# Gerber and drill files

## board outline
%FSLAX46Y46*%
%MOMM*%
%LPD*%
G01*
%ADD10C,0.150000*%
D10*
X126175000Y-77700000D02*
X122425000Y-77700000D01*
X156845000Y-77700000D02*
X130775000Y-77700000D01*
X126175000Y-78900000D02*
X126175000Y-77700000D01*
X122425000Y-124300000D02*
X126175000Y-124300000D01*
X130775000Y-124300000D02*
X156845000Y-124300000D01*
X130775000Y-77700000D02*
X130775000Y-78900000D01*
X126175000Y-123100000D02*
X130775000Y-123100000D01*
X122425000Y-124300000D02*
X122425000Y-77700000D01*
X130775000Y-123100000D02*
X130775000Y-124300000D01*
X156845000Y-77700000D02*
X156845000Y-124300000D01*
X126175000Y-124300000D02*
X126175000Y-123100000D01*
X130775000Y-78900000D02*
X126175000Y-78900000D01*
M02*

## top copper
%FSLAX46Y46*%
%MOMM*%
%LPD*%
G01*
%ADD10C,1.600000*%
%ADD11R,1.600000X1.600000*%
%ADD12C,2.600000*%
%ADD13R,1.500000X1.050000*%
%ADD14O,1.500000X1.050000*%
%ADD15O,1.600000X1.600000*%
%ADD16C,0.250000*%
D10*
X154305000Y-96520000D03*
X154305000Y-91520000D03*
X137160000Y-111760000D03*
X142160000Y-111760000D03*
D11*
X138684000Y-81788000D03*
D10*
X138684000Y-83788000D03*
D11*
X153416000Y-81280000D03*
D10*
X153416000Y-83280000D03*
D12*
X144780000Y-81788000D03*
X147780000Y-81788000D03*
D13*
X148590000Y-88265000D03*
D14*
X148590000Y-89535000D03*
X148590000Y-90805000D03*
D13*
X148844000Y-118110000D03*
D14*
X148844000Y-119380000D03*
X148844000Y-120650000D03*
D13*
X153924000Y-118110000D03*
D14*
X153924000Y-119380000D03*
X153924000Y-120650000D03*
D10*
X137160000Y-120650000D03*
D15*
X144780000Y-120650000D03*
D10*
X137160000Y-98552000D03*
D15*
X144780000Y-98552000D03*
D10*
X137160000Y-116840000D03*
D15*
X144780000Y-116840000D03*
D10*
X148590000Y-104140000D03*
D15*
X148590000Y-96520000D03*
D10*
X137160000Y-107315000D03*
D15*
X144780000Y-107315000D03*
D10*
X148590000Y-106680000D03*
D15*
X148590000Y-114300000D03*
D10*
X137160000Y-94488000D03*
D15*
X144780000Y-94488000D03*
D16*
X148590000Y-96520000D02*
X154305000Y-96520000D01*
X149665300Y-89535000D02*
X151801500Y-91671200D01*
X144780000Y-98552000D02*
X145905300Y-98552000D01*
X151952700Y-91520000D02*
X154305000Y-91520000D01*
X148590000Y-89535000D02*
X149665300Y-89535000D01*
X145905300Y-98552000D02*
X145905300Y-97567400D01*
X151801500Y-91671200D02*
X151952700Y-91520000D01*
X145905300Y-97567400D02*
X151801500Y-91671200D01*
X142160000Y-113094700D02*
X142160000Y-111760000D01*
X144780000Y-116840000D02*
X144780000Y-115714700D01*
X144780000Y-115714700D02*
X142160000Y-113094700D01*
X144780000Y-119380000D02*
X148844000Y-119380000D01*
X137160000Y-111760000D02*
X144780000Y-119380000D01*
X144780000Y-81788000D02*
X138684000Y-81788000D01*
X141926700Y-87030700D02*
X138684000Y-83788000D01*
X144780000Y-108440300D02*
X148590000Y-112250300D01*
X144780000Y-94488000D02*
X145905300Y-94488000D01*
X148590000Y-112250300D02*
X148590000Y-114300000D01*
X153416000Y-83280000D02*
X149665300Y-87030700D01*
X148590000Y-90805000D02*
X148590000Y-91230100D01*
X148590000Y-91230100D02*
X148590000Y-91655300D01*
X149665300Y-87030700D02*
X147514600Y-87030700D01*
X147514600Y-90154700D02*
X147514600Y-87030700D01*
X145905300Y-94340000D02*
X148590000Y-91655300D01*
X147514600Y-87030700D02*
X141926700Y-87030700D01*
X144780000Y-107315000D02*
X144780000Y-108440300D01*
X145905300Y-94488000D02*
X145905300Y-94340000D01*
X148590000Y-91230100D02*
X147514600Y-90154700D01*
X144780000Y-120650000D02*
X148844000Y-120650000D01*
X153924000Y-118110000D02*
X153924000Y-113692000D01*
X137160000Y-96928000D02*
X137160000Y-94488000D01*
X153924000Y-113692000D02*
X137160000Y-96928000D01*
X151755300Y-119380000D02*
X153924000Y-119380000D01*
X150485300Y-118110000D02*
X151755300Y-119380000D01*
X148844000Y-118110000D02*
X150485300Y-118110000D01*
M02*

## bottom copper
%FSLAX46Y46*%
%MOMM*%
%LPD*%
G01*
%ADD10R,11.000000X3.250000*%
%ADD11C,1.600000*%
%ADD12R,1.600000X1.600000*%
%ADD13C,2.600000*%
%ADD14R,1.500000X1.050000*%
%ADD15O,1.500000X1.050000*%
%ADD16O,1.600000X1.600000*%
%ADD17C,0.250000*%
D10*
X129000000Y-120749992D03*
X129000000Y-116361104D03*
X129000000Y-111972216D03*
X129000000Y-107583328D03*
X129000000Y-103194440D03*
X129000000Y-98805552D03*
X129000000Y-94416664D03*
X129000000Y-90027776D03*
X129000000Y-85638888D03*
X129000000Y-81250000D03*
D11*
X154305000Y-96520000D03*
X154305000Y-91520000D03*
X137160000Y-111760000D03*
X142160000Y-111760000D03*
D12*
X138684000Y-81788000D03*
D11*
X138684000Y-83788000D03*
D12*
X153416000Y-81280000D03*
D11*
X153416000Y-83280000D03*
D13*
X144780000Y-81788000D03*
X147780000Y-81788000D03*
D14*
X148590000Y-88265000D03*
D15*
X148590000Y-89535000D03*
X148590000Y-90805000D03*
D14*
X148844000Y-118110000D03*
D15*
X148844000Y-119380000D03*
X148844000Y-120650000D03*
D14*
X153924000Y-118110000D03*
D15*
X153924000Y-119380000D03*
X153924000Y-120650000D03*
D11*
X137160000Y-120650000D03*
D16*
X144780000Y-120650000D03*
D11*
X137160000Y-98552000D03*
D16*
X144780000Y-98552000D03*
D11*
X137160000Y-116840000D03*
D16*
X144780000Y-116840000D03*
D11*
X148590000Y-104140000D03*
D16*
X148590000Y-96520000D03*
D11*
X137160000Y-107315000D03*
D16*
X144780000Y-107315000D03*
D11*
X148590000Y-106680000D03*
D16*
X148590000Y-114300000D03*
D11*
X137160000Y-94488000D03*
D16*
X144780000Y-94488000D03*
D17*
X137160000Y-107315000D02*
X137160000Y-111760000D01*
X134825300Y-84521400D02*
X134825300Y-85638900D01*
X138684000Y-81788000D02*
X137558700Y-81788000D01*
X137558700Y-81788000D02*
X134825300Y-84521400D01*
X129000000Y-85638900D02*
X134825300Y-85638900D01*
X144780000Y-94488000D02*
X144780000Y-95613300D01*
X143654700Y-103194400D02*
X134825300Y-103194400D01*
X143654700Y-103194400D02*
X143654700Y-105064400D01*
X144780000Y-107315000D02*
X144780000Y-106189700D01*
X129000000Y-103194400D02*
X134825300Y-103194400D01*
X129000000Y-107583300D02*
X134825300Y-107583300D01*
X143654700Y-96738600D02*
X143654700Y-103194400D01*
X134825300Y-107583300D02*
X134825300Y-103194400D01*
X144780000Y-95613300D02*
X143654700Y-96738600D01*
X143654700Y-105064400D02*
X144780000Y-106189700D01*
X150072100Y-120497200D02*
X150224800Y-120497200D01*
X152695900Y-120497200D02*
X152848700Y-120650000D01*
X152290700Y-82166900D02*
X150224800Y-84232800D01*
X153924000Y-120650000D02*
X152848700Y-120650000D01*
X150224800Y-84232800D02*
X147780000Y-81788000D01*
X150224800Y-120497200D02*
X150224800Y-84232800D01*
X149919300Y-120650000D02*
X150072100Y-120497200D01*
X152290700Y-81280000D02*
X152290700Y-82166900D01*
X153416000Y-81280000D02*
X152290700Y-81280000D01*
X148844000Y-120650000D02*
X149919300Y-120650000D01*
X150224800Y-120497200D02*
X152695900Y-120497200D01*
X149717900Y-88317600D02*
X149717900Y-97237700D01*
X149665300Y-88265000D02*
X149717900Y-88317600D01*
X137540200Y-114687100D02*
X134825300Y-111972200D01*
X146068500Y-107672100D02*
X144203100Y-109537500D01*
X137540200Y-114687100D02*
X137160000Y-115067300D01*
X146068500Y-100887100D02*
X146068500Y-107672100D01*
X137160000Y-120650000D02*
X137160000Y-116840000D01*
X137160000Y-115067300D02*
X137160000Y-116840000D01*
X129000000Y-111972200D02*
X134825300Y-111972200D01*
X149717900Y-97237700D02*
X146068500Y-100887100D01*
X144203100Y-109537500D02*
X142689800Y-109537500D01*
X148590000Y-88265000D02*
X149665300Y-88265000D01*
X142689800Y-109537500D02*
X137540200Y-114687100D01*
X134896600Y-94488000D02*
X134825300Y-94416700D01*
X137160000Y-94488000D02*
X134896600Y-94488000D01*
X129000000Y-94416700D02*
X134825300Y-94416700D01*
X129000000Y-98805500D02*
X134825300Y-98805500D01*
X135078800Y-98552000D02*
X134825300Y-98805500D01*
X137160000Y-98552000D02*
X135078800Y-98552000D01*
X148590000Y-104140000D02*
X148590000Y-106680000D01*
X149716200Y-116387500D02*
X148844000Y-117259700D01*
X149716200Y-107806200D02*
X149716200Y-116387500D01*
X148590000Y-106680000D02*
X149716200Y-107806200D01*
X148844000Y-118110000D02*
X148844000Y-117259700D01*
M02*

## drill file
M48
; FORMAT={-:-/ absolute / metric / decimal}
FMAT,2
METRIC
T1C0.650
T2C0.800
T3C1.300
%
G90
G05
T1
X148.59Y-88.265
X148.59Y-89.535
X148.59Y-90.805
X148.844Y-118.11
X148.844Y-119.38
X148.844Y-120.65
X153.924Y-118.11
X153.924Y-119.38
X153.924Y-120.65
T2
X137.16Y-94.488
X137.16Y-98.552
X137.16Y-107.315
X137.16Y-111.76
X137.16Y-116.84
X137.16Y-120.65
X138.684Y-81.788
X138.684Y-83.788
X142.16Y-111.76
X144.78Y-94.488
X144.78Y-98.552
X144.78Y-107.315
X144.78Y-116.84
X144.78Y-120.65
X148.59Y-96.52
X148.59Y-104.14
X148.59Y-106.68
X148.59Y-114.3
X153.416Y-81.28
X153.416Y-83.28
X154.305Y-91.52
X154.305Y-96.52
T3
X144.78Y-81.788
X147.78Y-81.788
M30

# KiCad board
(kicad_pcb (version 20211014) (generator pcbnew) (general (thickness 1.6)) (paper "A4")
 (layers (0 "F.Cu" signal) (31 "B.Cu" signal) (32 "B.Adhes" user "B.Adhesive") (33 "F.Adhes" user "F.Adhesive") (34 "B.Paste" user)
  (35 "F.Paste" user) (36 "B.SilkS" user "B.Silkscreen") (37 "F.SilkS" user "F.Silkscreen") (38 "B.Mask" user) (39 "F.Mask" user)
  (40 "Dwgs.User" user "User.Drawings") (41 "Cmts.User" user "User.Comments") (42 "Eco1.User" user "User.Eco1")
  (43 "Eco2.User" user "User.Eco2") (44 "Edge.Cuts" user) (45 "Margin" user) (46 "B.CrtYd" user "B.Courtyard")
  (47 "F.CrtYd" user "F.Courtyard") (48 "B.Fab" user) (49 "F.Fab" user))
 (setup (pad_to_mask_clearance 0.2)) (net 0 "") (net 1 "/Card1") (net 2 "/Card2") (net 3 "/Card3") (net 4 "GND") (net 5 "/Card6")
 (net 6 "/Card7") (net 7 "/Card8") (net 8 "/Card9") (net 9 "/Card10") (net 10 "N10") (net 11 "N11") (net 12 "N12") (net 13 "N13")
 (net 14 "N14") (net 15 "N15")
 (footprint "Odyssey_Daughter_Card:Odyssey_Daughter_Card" (layer "F.Cu") (at 129 101)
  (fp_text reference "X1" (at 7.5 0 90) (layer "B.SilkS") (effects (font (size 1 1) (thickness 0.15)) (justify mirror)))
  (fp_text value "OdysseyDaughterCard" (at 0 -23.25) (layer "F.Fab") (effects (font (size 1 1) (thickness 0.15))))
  (pad "1" smd rect locked (at 0 19.749992) (size 11 3.25) (layers "B.Cu" "B.Mask") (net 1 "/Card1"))
  (pad "2" smd rect locked (at 0 15.361104) (size 11 3.25) (layers "B.Cu" "B.Mask") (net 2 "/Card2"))
  (pad "3" smd rect locked (at 0 10.972216) (size 11 3.25) (layers "B.Cu" "B.Mask") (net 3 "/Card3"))
  (pad "4" smd rect locked (at 0 6.583328) (size 11 3.25) (layers "B.Cu" "B.Mask") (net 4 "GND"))
  (pad "5" smd rect locked (at 0 2.19444) (size 11 3.25) (layers "B.Cu" "B.Mask") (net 4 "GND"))
  (pad "6" smd rect locked (at 0 -2.194448) (size 11 3.25) (layers "B.Cu" "B.Mask") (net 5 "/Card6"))
  (pad "7" smd rect locked (at 0 -6.583336) (size 11 3.25) (layers "B.Cu" "B.Mask") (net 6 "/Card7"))
  (pad "8" smd rect locked (at 0 -10.972224) (size 11 3.25) (layers "B.Cu" "B.Mask") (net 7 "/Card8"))
  (pad "9" smd rect locked (at 0 -15.361112) (size 11 3.25) (layers "B.Cu" "B.Mask") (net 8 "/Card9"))
  (pad "10" smd rect locked (at 0 -19.75) (size 11 3.25) (layers "B.Cu" "B.Mask") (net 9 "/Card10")))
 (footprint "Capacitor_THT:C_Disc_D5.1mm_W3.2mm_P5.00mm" (layer "F.Cu") (at 154.305 96.52 90)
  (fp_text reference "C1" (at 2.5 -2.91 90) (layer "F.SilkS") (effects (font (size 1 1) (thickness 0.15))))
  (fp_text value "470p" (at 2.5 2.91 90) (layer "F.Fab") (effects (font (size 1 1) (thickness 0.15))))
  (pad "1" thru_hole circle locked (at 0 0 90) (size 1.6 1.6) (drill 0.8) (layers *.Cu *.Mask) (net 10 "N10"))
  (pad "2" thru_hole circle locked (at 5 0 90) (size 1.6 1.6) (drill 0.8) (layers *.Cu *.Mask) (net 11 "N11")))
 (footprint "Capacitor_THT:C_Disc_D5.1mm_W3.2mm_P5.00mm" (layer "F.Cu") (at 137.16 111.76)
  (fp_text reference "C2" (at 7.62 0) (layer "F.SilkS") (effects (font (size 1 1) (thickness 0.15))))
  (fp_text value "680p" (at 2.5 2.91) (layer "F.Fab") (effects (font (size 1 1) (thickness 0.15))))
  (pad "1" thru_hole circle locked (at 0 0) (size 1.6 1.6) (drill 0.8) (layers *.Cu *.Mask) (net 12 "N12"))
  (pad "2" thru_hole circle locked (at 5 0) (size 1.6 1.6) (drill 0.8) (layers *.Cu *.Mask) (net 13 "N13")))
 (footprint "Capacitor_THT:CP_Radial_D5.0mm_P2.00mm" (layer "F.Cu") (at 138.684 81.788 -90)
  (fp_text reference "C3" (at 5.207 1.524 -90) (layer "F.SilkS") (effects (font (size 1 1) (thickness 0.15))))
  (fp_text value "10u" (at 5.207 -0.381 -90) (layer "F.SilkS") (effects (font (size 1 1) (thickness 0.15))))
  (pad "1" thru_hole rect locked (at 0 0 270) (size 1.6 1.6) (drill 0.8) (layers *.Cu *.Mask) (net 8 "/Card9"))
  (pad "2" thru_hole circle locked (at 2 0 270) (size 1.6 1.6) (drill 0.8) (layers *.Cu *.Mask) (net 4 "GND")))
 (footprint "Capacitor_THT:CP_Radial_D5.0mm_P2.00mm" (layer "F.Cu") (at 153.416 81.28 -90)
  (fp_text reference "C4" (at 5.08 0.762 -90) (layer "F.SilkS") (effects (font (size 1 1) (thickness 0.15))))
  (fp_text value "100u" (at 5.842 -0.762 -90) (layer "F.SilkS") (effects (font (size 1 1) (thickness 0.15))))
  (pad "1" thru_hole rect locked (at 0 0 270) (size 1.6 1.6) (drill 0.8) (layers *.Cu *.Mask) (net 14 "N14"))
  (pad "2" thru_hole circle locked (at 2 0 270) (size 1.6 1.6) (drill 0.8) (layers *.Cu *.Mask) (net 4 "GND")))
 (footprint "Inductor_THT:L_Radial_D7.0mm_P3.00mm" (layer "F.Cu") (at 144.78 81.788)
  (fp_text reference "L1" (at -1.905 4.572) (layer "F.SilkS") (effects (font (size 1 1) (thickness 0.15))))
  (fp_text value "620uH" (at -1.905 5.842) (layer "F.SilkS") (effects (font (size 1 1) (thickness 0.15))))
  (pad "1" thru_hole circle locked (at 0 0) (size 2.6 2.6) (drill 1.3) (layers *.Cu *.Mask) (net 8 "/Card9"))
  (pad "2" thru_hole circle locked (at 3 0) (size 2.6 2.6) (drill 1.3) (layers *.Cu *.Mask) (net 14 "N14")))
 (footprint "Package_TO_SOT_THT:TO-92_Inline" (layer "F.Cu") (at 148.59 88.265 -90)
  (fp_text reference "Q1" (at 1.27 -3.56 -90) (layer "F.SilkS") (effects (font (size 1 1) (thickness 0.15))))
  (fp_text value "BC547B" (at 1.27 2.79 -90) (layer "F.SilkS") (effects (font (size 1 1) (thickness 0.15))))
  (pad "1" thru_hole rect locked (at 0 0 270) (size 1.05 1.5) (drill 0.65) (layers *.Cu *.Mask) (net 3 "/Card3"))
  (pad "2" thru_hole oval locked (at 1.27 0 270) (size 1.05 1.5) (drill 0.65) (layers *.Cu *.Mask) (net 11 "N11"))
  (pad "3" thru_hole oval locked (at 2.54 0 270) (size 1.05 1.5) (drill 0.65) (layers *.Cu *.Mask) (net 4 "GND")))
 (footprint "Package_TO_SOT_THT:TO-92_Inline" (layer "F.Cu") (at 148.844 118.11 -90)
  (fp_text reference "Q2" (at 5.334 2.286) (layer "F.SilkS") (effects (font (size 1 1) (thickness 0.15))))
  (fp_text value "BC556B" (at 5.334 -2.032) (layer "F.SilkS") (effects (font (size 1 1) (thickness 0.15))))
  (pad "1" thru_hole rect locked (at 0 0 270) (size 1.05 1.5) (drill 0.65) (layers *.Cu *.Mask) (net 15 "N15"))
  (pad "2" thru_hole oval locked (at 1.27 0 270) (size 1.05 1.5) (drill 0.65) (layers *.Cu *.Mask) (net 12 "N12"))
  (pad "3" thru_hole oval locked (at 2.54 0 270) (size 1.05 1.5) (drill 0.65) (layers *.Cu *.Mask) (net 14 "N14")))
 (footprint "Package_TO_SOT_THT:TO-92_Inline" (layer "F.Cu") (at 153.924 118.11 -90)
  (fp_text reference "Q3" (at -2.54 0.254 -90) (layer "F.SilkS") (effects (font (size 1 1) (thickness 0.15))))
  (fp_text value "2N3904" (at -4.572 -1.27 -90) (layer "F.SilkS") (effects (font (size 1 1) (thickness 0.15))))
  (pad "1" thru_hole rect locked (at 0 0 270) (size 1.05 1.5) (drill 0.65) (layers *.Cu *.Mask) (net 6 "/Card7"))
  (pad "2" thru_hole oval locked (at 1.27 0 270) (size 1.05 1.5) (drill 0.65) (layers *.Cu *.Mask) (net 15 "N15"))
  (pad "3" thru_hole oval locked (at 2.54 0 270) (size 1.05 1.5) (drill 0.65) (layers *.Cu *.Mask) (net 14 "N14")))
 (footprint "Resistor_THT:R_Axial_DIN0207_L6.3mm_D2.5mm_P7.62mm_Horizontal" (layer "F.Cu") (at 137.16 120.65)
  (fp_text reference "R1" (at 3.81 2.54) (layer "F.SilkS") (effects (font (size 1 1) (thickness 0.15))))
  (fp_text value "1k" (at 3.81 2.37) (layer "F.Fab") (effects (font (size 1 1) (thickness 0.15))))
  (pad "1" thru_hole circle locked (at 0 0) (size 1.6 1.6) (drill 0.8) (layers *.Cu *.Mask) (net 3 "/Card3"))
  (pad "2" thru_hole oval locked (at 7.62 0) (size 1.6 1.6) (drill 0.8) (layers *.Cu *.Mask) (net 14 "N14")))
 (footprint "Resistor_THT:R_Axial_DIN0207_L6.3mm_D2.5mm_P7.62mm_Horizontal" (layer "F.Cu") (at 137.16 98.552)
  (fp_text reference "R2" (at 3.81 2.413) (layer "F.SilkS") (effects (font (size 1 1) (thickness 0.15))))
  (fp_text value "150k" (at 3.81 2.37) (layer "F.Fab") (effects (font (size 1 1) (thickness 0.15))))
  (pad "1" thru_hole circle locked (at 0 0) (size 1.6 1.6) (drill 0.8) (layers *.Cu *.Mask) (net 5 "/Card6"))
  (pad "2" thru_hole oval locked (at 7.62 0) (size 1.6 1.6) (drill 0.8) (layers *.Cu *.Mask) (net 11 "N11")))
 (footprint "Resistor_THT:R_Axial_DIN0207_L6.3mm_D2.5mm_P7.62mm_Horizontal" (layer "F.Cu") (at 137.16 116.84)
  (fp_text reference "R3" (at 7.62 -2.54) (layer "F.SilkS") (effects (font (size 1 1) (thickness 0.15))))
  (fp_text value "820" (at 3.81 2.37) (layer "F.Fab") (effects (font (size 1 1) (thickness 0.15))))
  (pad "1" thru_hole circle locked (at 0 0) (size 1.6 1.6) (drill 0.8) (layers *.Cu *.Mask) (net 3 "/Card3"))
  (pad "2" thru_hole oval locked (at 7.62 0) (size 1.6 1.6) (drill 0.8) (layers *.Cu *.Mask) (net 13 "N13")))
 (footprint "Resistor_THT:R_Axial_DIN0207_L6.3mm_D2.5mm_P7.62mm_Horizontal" (layer "F.Cu") (at 148.59 104.14 90)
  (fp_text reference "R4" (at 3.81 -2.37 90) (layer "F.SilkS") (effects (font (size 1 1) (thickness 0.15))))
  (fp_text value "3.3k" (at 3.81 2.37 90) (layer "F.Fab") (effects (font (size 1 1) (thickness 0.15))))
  (pad "1" thru_hole circle locked (at 0 0 90) (size 1.6 1.6) (drill 0.8) (layers *.Cu *.Mask) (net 15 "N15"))
  (pad "2" thru_hole oval locked (at 7.62 0 90) (size 1.6 1.6) (drill 0.8) (layers *.Cu *.Mask) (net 10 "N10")))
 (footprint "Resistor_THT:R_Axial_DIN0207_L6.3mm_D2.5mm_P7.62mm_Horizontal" (layer "F.Cu") (at 137.16 107.315)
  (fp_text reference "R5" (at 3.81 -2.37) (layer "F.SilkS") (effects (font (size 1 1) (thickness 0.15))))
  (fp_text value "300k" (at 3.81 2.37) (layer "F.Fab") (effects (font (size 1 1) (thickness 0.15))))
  (pad "1" thru_hole circle locked (at 0 0) (size 1.6 1.6) (drill 0.8) (layers *.Cu *.Mask) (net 12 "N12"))
  (pad "2" thru_hole oval locked (at 7.62 0) (size 1.6 1.6) (drill 0.8) (layers *.Cu *.Mask) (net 4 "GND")))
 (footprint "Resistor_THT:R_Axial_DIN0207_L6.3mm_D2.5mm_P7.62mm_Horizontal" (layer "F.Cu") (at 148.59 106.68 -90)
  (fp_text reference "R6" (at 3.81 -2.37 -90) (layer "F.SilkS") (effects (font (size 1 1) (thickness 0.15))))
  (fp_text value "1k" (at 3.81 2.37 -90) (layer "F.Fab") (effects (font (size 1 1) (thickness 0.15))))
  (pad "1" thru_hole circle locked (at 0 0 270) (size 1.6 1.6) (drill 0.8) (layers *.Cu *.Mask) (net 15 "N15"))
  (pad "2" thru_hole oval locked (at 7.62 0 270) (size 1.6 1.6) (drill 0.8) (layers *.Cu *.Mask) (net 4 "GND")))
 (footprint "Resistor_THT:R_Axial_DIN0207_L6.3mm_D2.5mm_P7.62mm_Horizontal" (layer "F.Cu") (at 137.16 94.488)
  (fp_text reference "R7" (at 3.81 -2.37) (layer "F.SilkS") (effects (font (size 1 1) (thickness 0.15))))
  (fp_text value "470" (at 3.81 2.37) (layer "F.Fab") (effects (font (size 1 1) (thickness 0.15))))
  (pad "1" thru_hole circle locked (at 0 0) (size 1.6 1.6) (drill 0.8) (layers *.Cu *.Mask) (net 6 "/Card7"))
  (pad "2" thru_hole oval locked (at 7.62 0) (size 1.6 1.6) (drill 0.8) (layers *.Cu *.Mask) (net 4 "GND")))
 (gr_line (start 126.175 77.7) (end 122.425 77.7) (layer "Edge.Cuts") (width 0.15))
 (gr_line (start 156.845 77.7) (end 130.775 77.7) (layer "Edge.Cuts") (width 0.15))
 (gr_line (start 126.175 78.9) (end 126.175 77.7) (layer "Edge.Cuts") (width 0.15))
 (gr_line (start 122.425 124.3) (end 126.175 124.3) (layer "Edge.Cuts") (width 0.15))
 (gr_line (start 130.775 124.3) (end 156.845 124.3) (layer "Edge.Cuts") (width 0.15))
 (gr_line (start 130.775 77.7) (end 130.775 78.9) (layer "Edge.Cuts") (width 0.15))
 (gr_line (start 126.175 123.1) (end 130.775 123.1) (layer "Edge.Cuts") (width 0.15))
 (gr_line (start 122.425 124.3) (end 122.425 77.7) (layer "Edge.Cuts") (width 0.15))
 (gr_line (start 130.775 123.1) (end 130.775 124.3) (layer "Edge.Cuts") (width 0.15))
 (gr_line (start 156.845 77.7) (end 156.845 124.3) (layer "Edge.Cuts") (width 0.15))
 (gr_line (start 126.175 124.3) (end 126.175 123.1) (layer "Edge.Cuts") (width 0.15))
 (gr_line (start 130.775 78.9) (end 126.175 78.9) (layer "Edge.Cuts") (width 0.15))
 (segment (start 148.59 96.52) (end 154.305 96.52) (width 0.25) (layer "F.Cu") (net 10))
 (segment (start 149.6653 89.535) (end 151.8015 91.6712) (width 0.25) (layer "F.Cu") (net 11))
 (segment (start 144.78 98.552) (end 145.9053 98.552) (width 0.25) (layer "F.Cu") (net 11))
 (segment (start 151.9527 91.52) (end 154.305 91.52) (width 0.25) (layer "F.Cu") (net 11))
 (segment (start 148.59 89.535) (end 149.6653 89.535) (width 0.25) (layer "F.Cu") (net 11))
 (segment (start 145.9053 98.552) (end 145.9053 97.5674) (width 0.25) (layer "F.Cu") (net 11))
 (segment (start 151.8015 91.6712) (end 151.9527 91.52) (width 0.25) (layer "F.Cu") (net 11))
 (segment (start 145.9053 97.5674) (end 151.8015 91.6712) (width 0.25) (layer "F.Cu") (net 11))
 (segment (start 142.16 113.0947) (end 142.16 111.76) (width 0.25) (layer "F.Cu") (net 13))
 (segment (start 144.78 116.84) (end 144.78 115.7147) (width 0.25) (layer "F.Cu") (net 13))
 (segment (start 144.78 115.7147) (end 142.16 113.0947) (width 0.25) (layer "F.Cu") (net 13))
 (segment (start 144.78 119.38) (end 148.844 119.38) (width 0.25) (layer "F.Cu") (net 12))
 (segment (start 137.16 111.76) (end 144.78 119.38) (width 0.25) (layer "F.Cu") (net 12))
 (segment (start 137.16 107.315) (end 137.16 111.76) (width 0.25) (layer "B.Cu") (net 12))
 (segment (start 144.78 81.788) (end 138.684 81.788) (width 0.25) (layer "F.Cu") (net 8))
 (segment (start 134.8253 84.5214) (end 134.8253 85.6389) (width 0.25) (layer "B.Cu") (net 8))
 (segment (start 138.684 81.788) (end 137.5587 81.788) (width 0.25) (layer "B.Cu") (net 8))
 (segment (start 137.5587 81.788) (end 134.8253 84.5214) (width 0.25) (layer "B.Cu") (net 8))
 (segment (start 129 85.6389) (end 134.8253 85.6389) (width 0.25) (layer "B.Cu") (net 8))
 (segment (start 141.9267 87.0307) (end 138.684 83.788) (width 0.25) (layer "F.Cu") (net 4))
 (segment (start 144.78 108.4403) (end 148.59 112.2503) (width 0.25) (layer "F.Cu") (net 4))
 (segment (start 144.78 94.488) (end 145.9053 94.488) (width 0.25) (layer "F.Cu") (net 4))
 (segment (start 148.59 112.2503) (end 148.59 114.3) (width 0.25) (layer "F.Cu") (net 4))
 (segment (start 153.416 83.28) (end 149.6653 87.0307) (width 0.25) (layer "F.Cu") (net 4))
 (segment (start 148.59 90.805) (end 148.59 91.2301) (width 0.25) (layer "F.Cu") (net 4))
 (segment (start 148.59 91.2301) (end 148.59 91.6553) (width 0.25) (layer "F.Cu") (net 4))
 (segment (start 149.6653 87.0307) (end 147.5146 87.0307) (width 0.25) (layer "F.Cu") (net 4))
 (segment (start 147.5146 90.1547) (end 147.5146 87.0307) (width 0.25) (layer "F.Cu") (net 4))
 (segment (start 145.9053 94.34) (end 148.59 91.6553) (width 0.25) (layer "F.Cu") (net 4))
 (segment (start 147.5146 87.0307) (end 141.9267 87.0307) (width 0.25) (layer "F.Cu") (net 4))
 (segment (start 144.78 107.315) (end 144.78 108.4403) (width 0.25) (layer "F.Cu") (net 4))
 (segment (start 145.9053 94.488) (end 145.9053 94.34) (width 0.25) (layer "F.Cu") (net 4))
 (segment (start 148.59 91.2301) (end 147.5146 90.1547) (width 0.25) (layer "F.Cu") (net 4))
 (segment (start 144.78 94.488) (end 144.78 95.6133) (width 0.25) (layer "B.Cu") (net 4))
 (segment (start 143.6547 103.1944) (end 134.8253 103.1944) (width 0.25) (layer "B.Cu") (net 4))
 (segment (start 143.6547 103.1944) (end 143.6547 105.0644) (width 0.25) (layer "B.Cu") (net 4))
 (segment (start 144.78 107.315) (end 144.78 106.1897) (width 0.25) (layer "B.Cu") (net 4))
 (segment (start 129 103.1944) (end 134.8253 103.1944) (width 0.25) (layer "B.Cu") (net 4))
 (segment (start 129 107.5833) (end 134.8253 107.5833) (width 0.25) (layer "B.Cu") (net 4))
 (segment (start 143.6547 96.7386) (end 143.6547 103.1944) (width 0.25) (layer "B.Cu") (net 4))
 (segment (start 134.8253 107.5833) (end 134.8253 103.1944) (width 0.25) (layer "B.Cu") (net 4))
 (segment (start 144.78 95.6133) (end 143.6547 96.7386) (width 0.25) (layer "B.Cu") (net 4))
 (segment (start 143.6547 105.0644) (end 144.78 106.1897) (width 0.25) (layer "B.Cu") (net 4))
 (segment (start 144.78 120.65) (end 148.844 120.65) (width 0.25) (layer "F.Cu") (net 14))
 (segment (start 150.0721 120.4972) (end 150.2248 120.4972) (width 0.25) (layer "B.Cu") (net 14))
 (segment (start 152.6959 120.4972) (end 152.8487 120.65) (width 0.25) (layer "B.Cu") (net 14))
 (segment (start 152.2907 82.1669) (end 150.2248 84.2328) (width 0.25) (layer "B.Cu") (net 14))
 (segment (start 153.924 120.65) (end 152.8487 120.65) (width 0.25) (layer "B.Cu") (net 14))
 (segment (start 150.2248 84.2328) (end 147.78 81.788) (width 0.25) (layer "B.Cu") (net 14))
 (segment (start 150.2248 120.4972) (end 150.2248 84.2328) (width 0.25) (layer "B.Cu") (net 14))
 (segment (start 149.9193 120.65) (end 150.0721 120.4972) (width 0.25) (layer "B.Cu") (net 14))
 (segment (start 152.2907 81.28) (end 152.2907 82.1669) (width 0.25) (layer "B.Cu") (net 14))
 (segment (start 153.416 81.28) (end 152.2907 81.28) (width 0.25) (layer "B.Cu") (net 14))
 (segment (start 148.844 120.65) (end 149.9193 120.65) (width 0.25) (layer "B.Cu") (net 14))
 (segment (start 150.2248 120.4972) (end 152.6959 120.4972) (width 0.25) (layer "B.Cu") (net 14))
 (segment (start 149.7179 88.3176) (end 149.7179 97.2377) (width 0.25) (layer "B.Cu") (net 3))
 (segment (start 149.6653 88.265) (end 149.7179 88.3176) (width 0.25) (layer "B.Cu") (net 3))
 (segment (start 137.5402 114.6871) (end 134.8253 111.9722) (width 0.25) (layer "B.Cu") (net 3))
 (segment (start 146.0685 107.6721) (end 144.2031 109.5375) (width 0.25) (layer "B.Cu") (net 3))
 (segment (start 137.5402 114.6871) (end 137.16 115.0673) (width 0.25) (layer "B.Cu") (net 3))
 (segment (start 146.0685 100.8871) (end 146.0685 107.6721) (width 0.25) (layer "B.Cu") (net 3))
 (segment (start 137.16 120.65) (end 137.16 116.84) (width 0.25) (layer "B.Cu") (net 3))
 (segment (start 137.16 115.0673) (end 137.16 116.84) (width 0.25) (layer "B.Cu") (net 3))
 (segment (start 129 111.9722) (end 134.8253 111.9722) (width 0.25) (layer "B.Cu") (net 3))
 (segment (start 149.7179 97.2377) (end 146.0685 100.8871) (width 0.25) (layer "B.Cu") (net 3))
 (segment (start 144.2031 109.5375) (end 142.6898 109.5375) (width 0.25) (layer "B.Cu") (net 3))
 (segment (start 148.59 88.265) (end 149.6653 88.265) (width 0.25) (layer "B.Cu") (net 3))
 (segment (start 142.6898 109.5375) (end 137.5402 114.6871) (width 0.25) (layer "B.Cu") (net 3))
 (segment (start 153.924 118.11) (end 153.924 113.692) (width 0.25) (layer "F.Cu") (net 6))
 (segment (start 137.16 96.928) (end 137.16 94.488) (width 0.25) (layer "F.Cu") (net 6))
 (segment (start 153.924 113.692) (end 137.16 96.928) (width 0.25) (layer "F.Cu") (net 6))
 (segment (start 134.8966 94.488) (end 134.8253 94.4167) (width 0.25) (layer "B.Cu") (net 6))
 (segment (start 137.16 94.488) (end 134.8966 94.488) (width 0.25) (layer "B.Cu") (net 6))
 (segment (start 129 94.4167) (end 134.8253 94.4167) (width 0.25) (layer "B.Cu") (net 6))
 (segment (start 129 98.8055) (end 134.8253 98.8055) (width 0.25) (layer "B.Cu") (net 5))
 (segment (start 135.0788 98.552) (end 134.8253 98.8055) (width 0.25) (layer "B.Cu") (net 5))
 (segment (start 137.16 98.552) (end 135.0788 98.552) (width 0.25) (layer "B.Cu") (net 5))
 (segment (start 151.7553 119.38) (end 153.924 119.38) (width 0.25) (layer "F.Cu") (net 15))
 (segment (start 150.4853 118.11) (end 151.7553 119.38) (width 0.25) (layer "F.Cu") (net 15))
 (segment (start 148.844 118.11) (end 150.4853 118.11) (width 0.25) (layer "F.Cu") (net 15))
 (segment (start 148.59 104.14) (end 148.59 106.68) (width 0.25) (layer "B.Cu") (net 15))
 (segment (start 149.7162 116.3875) (end 148.844 117.2597) (width 0.25) (layer "B.Cu") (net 15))
 (segment (start 149.7162 107.8062) (end 149.7162 116.3875) (width 0.25) (layer "B.Cu") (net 15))
 (segment (start 148.59 106.68) (end 149.7162 107.8062) (width 0.25) (layer "B.Cu") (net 15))
 (segment (start 148.844 118.11) (end 148.844 117.2597) (width 0.25) (layer "B.Cu") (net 15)))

